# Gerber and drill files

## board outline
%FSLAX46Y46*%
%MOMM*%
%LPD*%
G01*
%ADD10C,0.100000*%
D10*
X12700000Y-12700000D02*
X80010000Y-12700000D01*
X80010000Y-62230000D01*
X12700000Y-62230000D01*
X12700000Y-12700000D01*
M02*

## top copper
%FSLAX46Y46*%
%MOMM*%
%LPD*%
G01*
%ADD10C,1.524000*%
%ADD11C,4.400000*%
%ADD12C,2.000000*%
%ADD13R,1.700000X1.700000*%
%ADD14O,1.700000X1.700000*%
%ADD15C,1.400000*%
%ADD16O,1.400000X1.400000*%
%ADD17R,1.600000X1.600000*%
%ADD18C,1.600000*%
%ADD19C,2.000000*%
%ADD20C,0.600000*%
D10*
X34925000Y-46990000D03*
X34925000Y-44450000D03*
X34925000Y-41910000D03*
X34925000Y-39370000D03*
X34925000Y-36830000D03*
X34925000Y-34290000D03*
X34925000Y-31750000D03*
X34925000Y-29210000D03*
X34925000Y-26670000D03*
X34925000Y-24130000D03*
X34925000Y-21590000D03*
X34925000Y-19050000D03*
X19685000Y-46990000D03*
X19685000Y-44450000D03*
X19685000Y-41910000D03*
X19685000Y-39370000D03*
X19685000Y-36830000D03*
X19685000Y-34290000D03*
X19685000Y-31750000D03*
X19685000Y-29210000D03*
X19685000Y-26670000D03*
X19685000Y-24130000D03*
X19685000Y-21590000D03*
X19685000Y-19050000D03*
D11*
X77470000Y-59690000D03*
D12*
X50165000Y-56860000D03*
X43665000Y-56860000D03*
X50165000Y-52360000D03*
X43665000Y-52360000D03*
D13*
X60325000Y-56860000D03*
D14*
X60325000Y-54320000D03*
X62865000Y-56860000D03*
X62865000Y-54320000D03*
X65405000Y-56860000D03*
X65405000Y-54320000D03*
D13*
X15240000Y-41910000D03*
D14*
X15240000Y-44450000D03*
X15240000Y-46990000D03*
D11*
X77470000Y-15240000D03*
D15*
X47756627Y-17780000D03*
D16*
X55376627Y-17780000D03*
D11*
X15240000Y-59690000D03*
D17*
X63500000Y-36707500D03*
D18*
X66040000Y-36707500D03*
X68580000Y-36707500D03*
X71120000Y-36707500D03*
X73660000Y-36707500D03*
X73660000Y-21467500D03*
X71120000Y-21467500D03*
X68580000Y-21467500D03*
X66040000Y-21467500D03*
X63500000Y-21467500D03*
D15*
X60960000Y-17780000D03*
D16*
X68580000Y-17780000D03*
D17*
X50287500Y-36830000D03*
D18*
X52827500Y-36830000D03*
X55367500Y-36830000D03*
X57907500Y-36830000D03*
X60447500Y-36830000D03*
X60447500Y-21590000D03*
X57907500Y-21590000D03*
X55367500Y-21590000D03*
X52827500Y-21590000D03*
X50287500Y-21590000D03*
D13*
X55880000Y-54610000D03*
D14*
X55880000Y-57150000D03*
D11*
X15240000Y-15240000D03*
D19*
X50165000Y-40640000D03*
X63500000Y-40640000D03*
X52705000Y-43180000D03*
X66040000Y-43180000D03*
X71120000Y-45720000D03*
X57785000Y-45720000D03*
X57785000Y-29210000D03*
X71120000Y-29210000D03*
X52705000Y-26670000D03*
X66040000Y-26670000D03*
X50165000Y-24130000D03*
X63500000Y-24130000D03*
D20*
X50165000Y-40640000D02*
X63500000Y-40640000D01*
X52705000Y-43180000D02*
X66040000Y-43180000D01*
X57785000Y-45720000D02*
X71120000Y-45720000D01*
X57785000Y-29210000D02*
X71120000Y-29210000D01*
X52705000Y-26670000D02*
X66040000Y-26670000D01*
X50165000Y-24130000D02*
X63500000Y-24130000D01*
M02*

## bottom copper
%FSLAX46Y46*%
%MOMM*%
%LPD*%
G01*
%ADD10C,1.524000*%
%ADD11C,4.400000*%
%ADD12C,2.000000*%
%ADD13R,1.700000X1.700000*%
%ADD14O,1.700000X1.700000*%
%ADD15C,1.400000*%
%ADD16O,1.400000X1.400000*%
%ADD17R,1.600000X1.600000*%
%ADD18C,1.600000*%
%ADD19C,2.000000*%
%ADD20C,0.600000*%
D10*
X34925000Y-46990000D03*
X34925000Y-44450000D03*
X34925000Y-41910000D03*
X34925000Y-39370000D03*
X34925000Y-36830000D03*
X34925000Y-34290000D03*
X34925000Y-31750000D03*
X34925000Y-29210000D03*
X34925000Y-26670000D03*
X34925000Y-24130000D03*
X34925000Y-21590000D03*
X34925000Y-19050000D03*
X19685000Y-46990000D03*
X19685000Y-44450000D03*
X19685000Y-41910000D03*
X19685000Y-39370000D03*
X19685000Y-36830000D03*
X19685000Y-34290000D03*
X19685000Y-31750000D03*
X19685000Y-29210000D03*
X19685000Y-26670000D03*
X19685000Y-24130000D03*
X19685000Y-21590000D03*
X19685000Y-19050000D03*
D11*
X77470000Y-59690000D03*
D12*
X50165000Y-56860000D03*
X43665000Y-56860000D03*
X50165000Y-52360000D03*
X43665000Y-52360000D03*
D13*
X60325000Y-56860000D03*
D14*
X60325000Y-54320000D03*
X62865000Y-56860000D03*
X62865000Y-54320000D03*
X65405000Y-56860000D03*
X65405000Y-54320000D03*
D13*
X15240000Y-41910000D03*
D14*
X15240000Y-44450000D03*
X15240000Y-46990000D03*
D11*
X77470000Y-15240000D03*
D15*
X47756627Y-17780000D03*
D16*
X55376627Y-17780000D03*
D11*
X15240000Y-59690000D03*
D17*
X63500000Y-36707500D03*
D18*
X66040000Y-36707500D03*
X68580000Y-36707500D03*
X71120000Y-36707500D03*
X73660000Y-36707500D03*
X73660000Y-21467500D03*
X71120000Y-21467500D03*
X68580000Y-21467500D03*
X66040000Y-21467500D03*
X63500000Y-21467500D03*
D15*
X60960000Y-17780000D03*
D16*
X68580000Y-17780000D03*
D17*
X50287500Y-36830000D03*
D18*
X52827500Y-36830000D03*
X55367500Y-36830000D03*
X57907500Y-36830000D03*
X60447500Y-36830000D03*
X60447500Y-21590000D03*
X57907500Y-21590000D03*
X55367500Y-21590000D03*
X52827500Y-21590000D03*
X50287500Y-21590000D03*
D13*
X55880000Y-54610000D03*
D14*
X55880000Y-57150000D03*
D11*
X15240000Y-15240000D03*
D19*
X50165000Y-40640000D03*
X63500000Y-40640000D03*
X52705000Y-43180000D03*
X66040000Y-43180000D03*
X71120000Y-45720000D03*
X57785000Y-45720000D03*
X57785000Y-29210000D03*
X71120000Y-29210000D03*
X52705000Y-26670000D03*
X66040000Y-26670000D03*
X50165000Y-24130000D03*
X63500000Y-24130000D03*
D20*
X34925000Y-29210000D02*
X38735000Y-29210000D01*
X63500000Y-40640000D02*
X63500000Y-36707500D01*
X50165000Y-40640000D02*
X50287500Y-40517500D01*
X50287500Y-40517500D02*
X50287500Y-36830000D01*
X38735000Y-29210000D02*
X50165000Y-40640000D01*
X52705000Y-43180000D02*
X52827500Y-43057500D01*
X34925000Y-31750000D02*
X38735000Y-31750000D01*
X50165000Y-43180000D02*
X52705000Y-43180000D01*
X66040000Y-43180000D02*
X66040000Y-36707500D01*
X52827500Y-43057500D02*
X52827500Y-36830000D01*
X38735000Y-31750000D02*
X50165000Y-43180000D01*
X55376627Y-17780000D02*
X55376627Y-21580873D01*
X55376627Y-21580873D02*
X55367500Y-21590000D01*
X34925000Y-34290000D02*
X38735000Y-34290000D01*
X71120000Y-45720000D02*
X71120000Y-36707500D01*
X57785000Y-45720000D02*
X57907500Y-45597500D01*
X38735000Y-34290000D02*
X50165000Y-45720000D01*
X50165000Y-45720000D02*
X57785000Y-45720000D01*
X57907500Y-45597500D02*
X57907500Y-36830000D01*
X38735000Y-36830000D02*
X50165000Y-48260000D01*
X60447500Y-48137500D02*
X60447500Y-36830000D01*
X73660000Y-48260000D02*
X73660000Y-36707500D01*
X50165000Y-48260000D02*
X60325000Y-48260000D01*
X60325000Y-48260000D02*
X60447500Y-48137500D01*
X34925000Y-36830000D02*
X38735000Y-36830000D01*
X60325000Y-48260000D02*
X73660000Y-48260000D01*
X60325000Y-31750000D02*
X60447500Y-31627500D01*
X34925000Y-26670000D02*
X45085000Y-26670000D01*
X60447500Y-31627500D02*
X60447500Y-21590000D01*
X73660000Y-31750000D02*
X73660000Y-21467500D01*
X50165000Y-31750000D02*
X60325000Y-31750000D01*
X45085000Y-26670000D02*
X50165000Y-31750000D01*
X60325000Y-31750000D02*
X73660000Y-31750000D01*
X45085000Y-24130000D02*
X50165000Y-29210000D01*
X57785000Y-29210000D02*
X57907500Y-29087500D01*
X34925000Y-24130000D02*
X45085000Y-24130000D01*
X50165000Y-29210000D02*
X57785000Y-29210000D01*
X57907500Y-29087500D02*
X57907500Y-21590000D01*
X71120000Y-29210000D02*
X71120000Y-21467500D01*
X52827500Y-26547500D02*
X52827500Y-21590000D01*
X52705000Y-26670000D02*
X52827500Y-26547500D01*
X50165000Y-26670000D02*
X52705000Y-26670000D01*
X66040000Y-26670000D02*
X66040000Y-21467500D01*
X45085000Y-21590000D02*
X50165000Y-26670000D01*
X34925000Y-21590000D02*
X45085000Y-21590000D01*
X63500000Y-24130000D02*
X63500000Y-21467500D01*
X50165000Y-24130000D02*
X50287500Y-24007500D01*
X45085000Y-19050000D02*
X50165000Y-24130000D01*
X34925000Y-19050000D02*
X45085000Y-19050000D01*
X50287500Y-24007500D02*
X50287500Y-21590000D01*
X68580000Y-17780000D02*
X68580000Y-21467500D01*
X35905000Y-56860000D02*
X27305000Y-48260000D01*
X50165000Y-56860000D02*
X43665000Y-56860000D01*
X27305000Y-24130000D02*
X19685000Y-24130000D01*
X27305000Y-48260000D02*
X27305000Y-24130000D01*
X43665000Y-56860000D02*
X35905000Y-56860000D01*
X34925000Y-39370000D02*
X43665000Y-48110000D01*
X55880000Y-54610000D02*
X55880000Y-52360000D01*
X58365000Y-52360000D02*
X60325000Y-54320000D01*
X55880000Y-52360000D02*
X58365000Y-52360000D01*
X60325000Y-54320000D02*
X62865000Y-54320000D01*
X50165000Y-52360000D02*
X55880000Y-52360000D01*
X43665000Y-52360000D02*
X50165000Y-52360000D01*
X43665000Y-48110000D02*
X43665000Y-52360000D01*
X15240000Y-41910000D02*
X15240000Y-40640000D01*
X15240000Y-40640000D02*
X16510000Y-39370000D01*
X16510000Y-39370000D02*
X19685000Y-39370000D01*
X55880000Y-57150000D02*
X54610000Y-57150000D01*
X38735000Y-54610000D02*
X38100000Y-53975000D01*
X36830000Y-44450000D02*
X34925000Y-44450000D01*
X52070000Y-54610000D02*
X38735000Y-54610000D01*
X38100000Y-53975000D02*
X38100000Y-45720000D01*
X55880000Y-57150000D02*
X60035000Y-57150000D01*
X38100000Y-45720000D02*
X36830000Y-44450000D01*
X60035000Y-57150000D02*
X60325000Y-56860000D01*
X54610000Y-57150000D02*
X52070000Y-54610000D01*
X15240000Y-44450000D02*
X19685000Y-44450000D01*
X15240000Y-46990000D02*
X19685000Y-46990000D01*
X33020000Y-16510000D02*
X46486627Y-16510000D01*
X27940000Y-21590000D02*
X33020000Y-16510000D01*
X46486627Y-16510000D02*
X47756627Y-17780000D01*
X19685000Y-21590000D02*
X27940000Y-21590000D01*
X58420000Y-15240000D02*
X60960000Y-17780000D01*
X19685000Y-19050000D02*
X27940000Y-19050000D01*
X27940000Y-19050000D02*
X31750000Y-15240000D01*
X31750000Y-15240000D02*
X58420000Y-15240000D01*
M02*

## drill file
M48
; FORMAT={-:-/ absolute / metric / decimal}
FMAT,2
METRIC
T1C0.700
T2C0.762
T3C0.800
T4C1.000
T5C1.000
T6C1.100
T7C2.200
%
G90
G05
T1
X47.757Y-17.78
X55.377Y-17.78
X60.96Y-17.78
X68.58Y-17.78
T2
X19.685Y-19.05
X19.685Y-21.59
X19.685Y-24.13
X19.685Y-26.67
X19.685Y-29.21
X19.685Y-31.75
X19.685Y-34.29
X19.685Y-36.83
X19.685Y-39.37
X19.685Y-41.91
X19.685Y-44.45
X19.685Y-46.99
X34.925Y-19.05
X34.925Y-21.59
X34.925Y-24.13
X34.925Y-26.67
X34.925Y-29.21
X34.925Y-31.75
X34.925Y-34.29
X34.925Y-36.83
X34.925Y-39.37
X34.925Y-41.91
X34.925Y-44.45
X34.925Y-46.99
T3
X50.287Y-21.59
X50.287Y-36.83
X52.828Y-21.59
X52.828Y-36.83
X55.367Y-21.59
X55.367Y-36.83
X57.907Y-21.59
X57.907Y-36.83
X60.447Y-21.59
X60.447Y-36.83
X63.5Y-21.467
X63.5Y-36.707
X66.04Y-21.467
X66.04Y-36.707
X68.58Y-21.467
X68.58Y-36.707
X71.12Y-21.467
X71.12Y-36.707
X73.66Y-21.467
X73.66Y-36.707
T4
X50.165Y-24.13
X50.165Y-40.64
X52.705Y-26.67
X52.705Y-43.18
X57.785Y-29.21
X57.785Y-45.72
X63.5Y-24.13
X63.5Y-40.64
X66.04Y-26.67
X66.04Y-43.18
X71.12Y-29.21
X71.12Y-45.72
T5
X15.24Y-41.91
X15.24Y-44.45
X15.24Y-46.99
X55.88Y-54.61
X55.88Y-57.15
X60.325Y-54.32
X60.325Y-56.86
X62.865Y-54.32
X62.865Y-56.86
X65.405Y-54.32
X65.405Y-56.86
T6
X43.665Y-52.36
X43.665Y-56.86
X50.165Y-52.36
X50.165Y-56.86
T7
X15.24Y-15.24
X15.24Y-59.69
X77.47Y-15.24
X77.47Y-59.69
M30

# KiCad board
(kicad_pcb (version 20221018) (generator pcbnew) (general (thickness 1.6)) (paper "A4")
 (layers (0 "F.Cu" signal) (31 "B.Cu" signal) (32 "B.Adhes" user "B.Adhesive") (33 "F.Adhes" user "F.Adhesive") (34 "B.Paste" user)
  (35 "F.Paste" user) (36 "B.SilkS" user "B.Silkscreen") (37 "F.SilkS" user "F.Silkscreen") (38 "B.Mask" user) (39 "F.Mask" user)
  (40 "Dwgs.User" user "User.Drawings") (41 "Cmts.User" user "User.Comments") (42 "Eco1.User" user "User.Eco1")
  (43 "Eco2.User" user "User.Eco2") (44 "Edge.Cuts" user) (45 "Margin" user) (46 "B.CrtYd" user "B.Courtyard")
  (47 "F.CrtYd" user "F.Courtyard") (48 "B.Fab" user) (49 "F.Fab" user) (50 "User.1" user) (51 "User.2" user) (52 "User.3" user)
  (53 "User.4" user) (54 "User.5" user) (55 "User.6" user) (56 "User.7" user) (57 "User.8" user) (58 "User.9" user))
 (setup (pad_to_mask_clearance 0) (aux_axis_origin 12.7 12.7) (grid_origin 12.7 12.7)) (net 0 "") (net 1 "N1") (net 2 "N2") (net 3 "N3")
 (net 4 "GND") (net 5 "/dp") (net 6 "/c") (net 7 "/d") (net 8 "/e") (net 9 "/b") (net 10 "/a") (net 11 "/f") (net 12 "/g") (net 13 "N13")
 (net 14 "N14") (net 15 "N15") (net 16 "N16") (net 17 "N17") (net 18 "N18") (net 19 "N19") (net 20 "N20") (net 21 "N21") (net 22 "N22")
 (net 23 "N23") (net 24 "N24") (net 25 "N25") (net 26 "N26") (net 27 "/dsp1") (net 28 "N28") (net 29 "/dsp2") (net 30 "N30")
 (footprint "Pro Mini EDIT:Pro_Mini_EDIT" (layer "F.Cu") (at 34.925 46.99 180)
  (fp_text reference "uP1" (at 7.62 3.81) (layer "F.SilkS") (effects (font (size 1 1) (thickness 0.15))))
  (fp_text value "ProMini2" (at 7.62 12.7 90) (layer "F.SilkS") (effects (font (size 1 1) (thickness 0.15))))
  (pad "7" thru_hole circle (at 0 0 180) (size 1.524 1.524) (drill 0.762) (layers "*.Cu" "*.Mask" "F.SilkS") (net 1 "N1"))
  (pad "8" thru_hole circle (at 0 2.54 180) (size 1.524 1.524) (drill 0.762) (layers "*.Cu" "*.Mask" "F.SilkS") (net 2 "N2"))
  (pad "9" thru_hole circle (at 0 5.08 180) (size 1.524 1.524) (drill 0.762) (layers "*.Cu" "*.Mask" "F.SilkS") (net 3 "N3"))
  (pad "10" thru_hole circle (at 0 7.62 180) (size 1.524 1.524) (drill 0.762) (layers "*.Cu" "*.Mask" "F.SilkS") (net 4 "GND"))
  (pad "11" thru_hole circle (at 0 10.16 180) (size 1.524 1.524) (drill 0.762) (layers "*.Cu" "*.Mask" "F.SilkS") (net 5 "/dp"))
  (pad "12" thru_hole circle (at 0 12.7 180) (size 1.524 1.524) (drill 0.762) (layers "*.Cu" "*.Mask" "F.SilkS") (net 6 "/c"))
  (pad "13" thru_hole circle (at 0 15.24 180) (size 1.524 1.524) (drill 0.762) (layers "*.Cu" "*.Mask" "F.SilkS") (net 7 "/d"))
  (pad "14" thru_hole circle (at 0 17.78 180) (size 1.524 1.524) (drill 0.762) (layers "*.Cu" "*.Mask" "F.SilkS") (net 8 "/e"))
  (pad "15" thru_hole circle (at 0 20.32 180) (size 1.524 1.524) (drill 0.762) (layers "*.Cu" "*.Mask" "F.SilkS") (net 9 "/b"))
  (pad "16" thru_hole circle (at 0 22.86 180) (size 1.524 1.524) (drill 0.762) (layers "*.Cu" "*.Mask" "F.SilkS") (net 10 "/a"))
  (pad "17" thru_hole circle (at 0 25.4 180) (size 1.524 1.524) (drill 0.762) (layers "*.Cu" "*.Mask" "F.SilkS") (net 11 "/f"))
  (pad "18" thru_hole circle (at 0 27.94 180) (size 1.524 1.524) (drill 0.762) (layers "*.Cu" "*.Mask" "F.SilkS") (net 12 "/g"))
  (pad "19" thru_hole circle (at 15.24 0 180) (size 1.524 1.524) (drill 0.762) (layers "*.Cu" "*.Mask" "F.SilkS") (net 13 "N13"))
  (pad "20" thru_hole circle (at 15.24 2.54 180) (size 1.524 1.524) (drill 0.762) (layers "*.Cu" "*.Mask" "F.SilkS") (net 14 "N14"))
  (pad "21" thru_hole circle (at 15.24 5.08 180) (size 1.524 1.524) (drill 0.762) (layers "*.Cu" "*.Mask" "F.SilkS") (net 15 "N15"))
  (pad "22" thru_hole circle (at 15.24 7.62 180) (size 1.524 1.524) (drill 0.762) (layers "*.Cu" "*.Mask" "F.SilkS") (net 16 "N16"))
  (pad "23" thru_hole circle (at 15.24 10.16 180) (size 1.524 1.524) (drill 0.762) (layers "*.Cu" "*.Mask" "F.SilkS") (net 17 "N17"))
  (pad "24" thru_hole circle (at 15.24 12.7 180) (size 1.524 1.524) (drill 0.762) (layers "*.Cu" "*.Mask" "F.SilkS") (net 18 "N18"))
  (pad "25" thru_hole circle (at 15.24 15.24 180) (size 1.524 1.524) (drill 0.762) (layers "*.Cu" "*.Mask" "F.SilkS") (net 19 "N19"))
  (pad "26" thru_hole circle (at 15.24 17.78 180) (size 1.524 1.524) (drill 0.762) (layers "*.Cu" "*.Mask" "F.SilkS") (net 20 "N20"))
  (pad "27" thru_hole circle (at 15.24 20.32 180) (size 1.524 1.524) (drill 0.762) (layers "*.Cu" "*.Mask" "F.SilkS") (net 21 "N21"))
  (pad "28" thru_hole circle (at 15.24 22.86 180) (size 1.524 1.524) (drill 0.762) (layers "*.Cu" "*.Mask" "F.SilkS") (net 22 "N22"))
  (pad "29" thru_hole circle (at 15.24 25.4 180) (size 1.524 1.524) (drill 0.762) (layers "*.Cu" "*.Mask" "F.SilkS") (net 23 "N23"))
  (pad "30" thru_hole circle (at 15.24 27.94 180) (size 1.524 1.524) (drill 0.762) (layers "*.Cu" "*.Mask" "F.SilkS") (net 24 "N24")))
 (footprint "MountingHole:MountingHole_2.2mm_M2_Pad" (layer "F.Cu") (at 77.47 59.69)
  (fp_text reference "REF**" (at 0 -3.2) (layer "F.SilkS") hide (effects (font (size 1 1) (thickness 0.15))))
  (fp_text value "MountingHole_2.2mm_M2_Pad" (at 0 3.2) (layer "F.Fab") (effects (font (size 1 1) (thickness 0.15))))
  (pad "1" thru_hole circle (at 0 0) (size 4.4 4.4) (drill 2.2) (layers "*.Cu" "*.Mask")))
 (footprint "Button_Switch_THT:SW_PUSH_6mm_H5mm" (layer "F.Cu") (at 50.165 56.86 180)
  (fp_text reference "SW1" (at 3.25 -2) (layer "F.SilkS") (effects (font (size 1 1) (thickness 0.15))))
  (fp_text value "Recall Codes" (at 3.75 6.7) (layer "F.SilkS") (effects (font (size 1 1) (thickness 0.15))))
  (pad "1" thru_hole circle (at 0 0 270) (size 2 2) (drill 1.1) (layers "*.Cu" "*.Mask") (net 22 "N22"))
  (pad "1" thru_hole circle (at 6.5 0 270) (size 2 2) (drill 1.1) (layers "*.Cu" "*.Mask") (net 22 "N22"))
  (pad "2" thru_hole circle (at 0 4.5 270) (size 2 2) (drill 1.1) (layers "*.Cu" "*.Mask") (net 4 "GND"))
  (pad "2" thru_hole circle (at 6.5 4.5 270) (size 2 2) (drill 1.1) (layers "*.Cu" "*.Mask") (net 4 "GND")))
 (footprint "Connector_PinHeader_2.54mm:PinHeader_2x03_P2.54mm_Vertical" (layer "F.Cu") (at 60.325 56.86 90)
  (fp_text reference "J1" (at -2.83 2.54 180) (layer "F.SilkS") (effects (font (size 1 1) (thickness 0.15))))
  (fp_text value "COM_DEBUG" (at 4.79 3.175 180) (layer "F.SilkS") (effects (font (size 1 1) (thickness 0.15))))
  (pad "1" thru_hole rect (at 0 0 90) (size 1.7 1.7) (drill 1) (layers "*.Cu" "*.Mask") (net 2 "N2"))
  (pad "2" thru_hole oval (at 2.54 0 90) (size 1.7 1.7) (drill 1) (layers "*.Cu" "*.Mask") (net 4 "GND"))
  (pad "3" thru_hole oval (at 0 2.54 90) (size 1.7 1.7) (drill 1) (layers "*.Cu" "*.Mask"))
  (pad "4" thru_hole oval (at 2.54 2.54 90) (size 1.7 1.7) (drill 1) (layers "*.Cu" "*.Mask") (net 4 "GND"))
  (pad "5" thru_hole oval (at 0 5.08 90) (size 1.7 1.7) (drill 1) (layers "*.Cu" "*.Mask") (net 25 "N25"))
  (pad "6" thru_hole oval (at 2.54 5.08 90) (size 1.7 1.7) (drill 1) (layers "*.Cu" "*.Mask") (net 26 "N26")))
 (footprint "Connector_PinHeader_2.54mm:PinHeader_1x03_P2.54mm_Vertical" (layer "F.Cu") (at 15.24 41.91)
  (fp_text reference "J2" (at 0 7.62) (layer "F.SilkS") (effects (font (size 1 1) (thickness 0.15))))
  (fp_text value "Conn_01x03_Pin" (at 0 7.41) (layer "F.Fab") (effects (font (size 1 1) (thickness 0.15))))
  (pad "1" thru_hole rect (at 0 0) (size 1.7 1.7) (drill 1) (layers "*.Cu" "*.Mask") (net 16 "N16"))
  (pad "2" thru_hole oval (at 0 2.54) (size 1.7 1.7) (drill 1) (layers "*.Cu" "*.Mask") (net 14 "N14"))
  (pad "3" thru_hole oval (at 0 5.08) (size 1.7 1.7) (drill 1) (layers "*.Cu" "*.Mask") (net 13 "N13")))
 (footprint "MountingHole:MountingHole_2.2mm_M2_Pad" (layer "F.Cu") (at 77.47 15.24)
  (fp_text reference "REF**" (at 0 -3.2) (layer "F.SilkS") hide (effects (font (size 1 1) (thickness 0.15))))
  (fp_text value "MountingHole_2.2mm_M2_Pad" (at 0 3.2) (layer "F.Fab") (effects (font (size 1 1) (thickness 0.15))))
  (pad "1" thru_hole circle (at 0 0) (size 4.4 4.4) (drill 2.2) (layers "*.Cu" "*.Mask")))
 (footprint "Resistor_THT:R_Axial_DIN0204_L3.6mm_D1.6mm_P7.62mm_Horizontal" (layer "F.Cu") (at 47.756627 17.78)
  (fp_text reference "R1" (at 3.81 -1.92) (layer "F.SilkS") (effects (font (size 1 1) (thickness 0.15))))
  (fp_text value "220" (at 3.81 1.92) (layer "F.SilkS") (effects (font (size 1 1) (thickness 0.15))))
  (pad "1" thru_hole circle (at 0 0) (size 1.4 1.4) (drill 0.7) (layers "*.Cu" "*.Mask") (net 23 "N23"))
  (pad "2" thru_hole oval (at 7.62 0) (size 1.4 1.4) (drill 0.7) (layers "*.Cu" "*.Mask") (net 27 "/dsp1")))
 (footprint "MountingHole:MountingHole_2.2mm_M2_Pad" (layer "F.Cu") (at 15.24 59.69)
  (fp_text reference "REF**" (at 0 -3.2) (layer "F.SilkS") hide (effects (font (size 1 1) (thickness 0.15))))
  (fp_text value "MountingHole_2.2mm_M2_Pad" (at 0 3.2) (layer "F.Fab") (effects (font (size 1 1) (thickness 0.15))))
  (pad "1" thru_hole circle (at 0 0) (size 4.4 4.4) (drill 2.2) (layers "*.Cu" "*.Mask")))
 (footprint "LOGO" (layer "F.Cu") (at 25.4 58.42)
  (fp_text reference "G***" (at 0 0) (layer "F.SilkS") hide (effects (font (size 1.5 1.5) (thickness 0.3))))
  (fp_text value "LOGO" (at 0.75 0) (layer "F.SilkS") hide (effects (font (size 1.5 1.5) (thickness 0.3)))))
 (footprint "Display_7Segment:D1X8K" (layer "F.Cu") (at 63.5 36.7075 90)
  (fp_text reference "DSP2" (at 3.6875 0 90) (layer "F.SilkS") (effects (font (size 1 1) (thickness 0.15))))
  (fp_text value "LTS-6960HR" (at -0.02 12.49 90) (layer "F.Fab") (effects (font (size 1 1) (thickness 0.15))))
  (pad "1" thru_hole rect (at 0 0) (size 1.6 1.6) (drill 0.8) (layers "*.Cu" "*.Mask") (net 8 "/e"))
  (pad "2" thru_hole circle (at 0 2.54) (size 1.6 1.6) (drill 0.8) (layers "*.Cu" "*.Mask") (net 7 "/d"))
  (pad "3" thru_hole circle (at 0 5.08) (size 1.6 1.6) (drill 0.8) (layers "*.Cu" "*.Mask") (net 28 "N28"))
  (pad "4" thru_hole circle (at 0 7.62) (size 1.6 1.6) (drill 0.8) (layers "*.Cu" "*.Mask") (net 6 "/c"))
  (pad "5" thru_hole circle (at 0 10.16) (size 1.6 1.6) (drill 0.8) (layers "*.Cu" "*.Mask") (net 5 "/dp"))
  (pad "6" thru_hole circle (at 15.24 10.16) (size 1.6 1.6) (drill 0.8) (layers "*.Cu" "*.Mask") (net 9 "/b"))
  (pad "7" thru_hole circle (at 15.24 7.62) (size 1.6 1.6) (drill 0.8) (layers "*.Cu" "*.Mask") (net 10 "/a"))
  (pad "8" thru_hole circle (at 15.24 5.08) (size 1.6 1.6) (drill 0.8) (layers "*.Cu" "*.Mask") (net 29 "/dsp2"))
  (pad "9" thru_hole circle (at 15.24 2.54) (size 1.6 1.6) (drill 0.8) (layers "*.Cu" "*.Mask") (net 11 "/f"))
  (pad "10" thru_hole circle (at 15.24 0) (size 1.6 1.6) (drill 0.8) (layers "*.Cu" "*.Mask") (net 12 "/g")))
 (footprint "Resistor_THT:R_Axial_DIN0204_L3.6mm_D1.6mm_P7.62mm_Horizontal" (layer "F.Cu") (at 60.96 17.78)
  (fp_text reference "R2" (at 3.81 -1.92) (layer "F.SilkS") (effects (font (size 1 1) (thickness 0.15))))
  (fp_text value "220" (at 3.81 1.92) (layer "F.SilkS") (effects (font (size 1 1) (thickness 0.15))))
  (pad "1" thru_hole circle (at 0 0) (size 1.4 1.4) (drill 0.7) (layers "*.Cu" "*.Mask") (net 24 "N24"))
  (pad "2" thru_hole oval (at 7.62 0) (size 1.4 1.4) (drill 0.7) (layers "*.Cu" "*.Mask") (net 29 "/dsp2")))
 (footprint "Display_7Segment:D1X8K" (layer "F.Cu") (at 50.2875 36.83 90)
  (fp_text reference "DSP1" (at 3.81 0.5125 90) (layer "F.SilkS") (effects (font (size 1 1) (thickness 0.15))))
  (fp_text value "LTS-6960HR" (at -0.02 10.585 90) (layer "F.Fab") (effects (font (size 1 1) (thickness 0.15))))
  (pad "1" thru_hole rect (at 0 0) (size 1.6 1.6) (drill 0.8) (layers "*.Cu" "*.Mask") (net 8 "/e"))
  (pad "2" thru_hole circle (at 0 2.54) (size 1.6 1.6) (drill 0.8) (layers "*.Cu" "*.Mask") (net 7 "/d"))
  (pad "3" thru_hole circle (at 0 5.08) (size 1.6 1.6) (drill 0.8) (layers "*.Cu" "*.Mask") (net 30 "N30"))
  (pad "4" thru_hole circle (at 0 7.62) (size 1.6 1.6) (drill 0.8) (layers "*.Cu" "*.Mask") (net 6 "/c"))
  (pad "5" thru_hole circle (at 0 10.16) (size 1.6 1.6) (drill 0.8) (layers "*.Cu" "*.Mask") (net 5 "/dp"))
  (pad "6" thru_hole circle (at 15.24 10.16) (size 1.6 1.6) (drill 0.8) (layers "*.Cu" "*.Mask") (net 9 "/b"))
  (pad "7" thru_hole circle (at 15.24 7.62) (size 1.6 1.6) (drill 0.8) (layers "*.Cu" "*.Mask") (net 10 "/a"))
  (pad "8" thru_hole circle (at 15.24 5.08) (size 1.6 1.6) (drill 0.8) (layers "*.Cu" "*.Mask") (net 27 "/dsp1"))
  (pad "9" thru_hole circle (at 15.24 2.54) (size 1.6 1.6) (drill 0.8) (layers "*.Cu" "*.Mask") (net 11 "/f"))
  (pad "10" thru_hole circle (at 15.24 0) (size 1.6 1.6) (drill 0.8) (layers "*.Cu" "*.Mask") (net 12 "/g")))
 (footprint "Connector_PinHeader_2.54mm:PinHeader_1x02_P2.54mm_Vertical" (layer "F.Cu") (at 55.88 54.61)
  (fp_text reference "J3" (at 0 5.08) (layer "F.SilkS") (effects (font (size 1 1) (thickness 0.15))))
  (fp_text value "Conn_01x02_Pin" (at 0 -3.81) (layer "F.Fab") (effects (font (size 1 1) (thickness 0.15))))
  (pad "1" thru_hole rect (at 0 0) (size 1.7 1.7) (drill 1) (layers "*.Cu" "*.Mask") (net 4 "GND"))
  (pad "2" thru_hole oval (at 0 2.54) (size 1.7 1.7) (drill 1) (layers "*.Cu" "*.Mask") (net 2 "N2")))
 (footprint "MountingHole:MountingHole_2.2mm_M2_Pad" (layer "F.Cu") (at 15.24 15.24)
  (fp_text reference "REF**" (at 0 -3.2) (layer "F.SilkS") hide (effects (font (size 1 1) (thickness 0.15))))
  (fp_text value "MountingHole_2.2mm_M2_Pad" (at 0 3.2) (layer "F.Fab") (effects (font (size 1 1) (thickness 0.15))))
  (pad "1" thru_hole circle (at 0 0) (size 4.4 4.4) (drill 2.2) (layers "*.Cu" "*.Mask")))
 (gr_rect (start 12.7 12.7) (end 80.01 62.23) (stroke (width 0.1) (type default)) (fill none) (layer "Edge.Cuts"))
 (segment (start 50.165 40.64) (end 63.5 40.64) (width 0.6) (layer "F.Cu") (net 8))
 (via (at 50.165 40.64) (size 2) (drill 1) (layers "F.Cu" "B.Cu") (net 8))
 (via (at 63.5 40.64) (size 2) (drill 1) (layers "F.Cu" "B.Cu") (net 8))
 (segment (start 34.925 29.21) (end 38.735 29.21) (width 0.6) (layer "B.Cu") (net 8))
 (segment (start 63.5 40.64) (end 63.5 36.7075) (width 0.6) (layer "B.Cu") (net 8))
 (segment (start 50.165 40.64) (end 50.2875 40.5175) (width 0.6) (layer "B.Cu") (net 8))
 (segment (start 50.2875 40.5175) (end 50.2875 36.83) (width 0.6) (layer "B.Cu") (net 8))
 (segment (start 38.735 29.21) (end 50.165 40.64) (width 0.6) (layer "B.Cu") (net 8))
 (segment (start 52.705 43.18) (end 66.04 43.18) (width 0.6) (layer "F.Cu") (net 7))
 (via (at 52.705 43.18) (size 2) (drill 1) (layers "F.Cu" "B.Cu") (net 7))
 (via (at 66.04 43.18) (size 2) (drill 1) (layers "F.Cu" "B.Cu") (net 7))
 (segment (start 52.705 43.18) (end 52.8275 43.0575) (width 0.6) (layer "B.Cu") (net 7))
 (segment (start 34.925 31.75) (end 38.735 31.75) (width 0.6) (layer "B.Cu") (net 7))
 (segment (start 50.165 43.18) (end 52.705 43.18) (width 0.6) (layer "B.Cu") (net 7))
 (segment (start 66.04 43.18) (end 66.04 36.7075) (width 0.6) (layer "B.Cu") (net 7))
 (segment (start 52.8275 43.0575) (end 52.8275 36.83) (width 0.6) (layer "B.Cu") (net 7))
 (segment (start 38.735 31.75) (end 50.165 43.18) (width 0.6) (layer "B.Cu") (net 7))
 (segment (start 55.376627 17.78) (end 55.376627 21.580873) (width 0.6) (layer "B.Cu") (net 27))
 (segment (start 55.376627 21.580873) (end 55.3675 21.59) (width 0.6) (layer "B.Cu") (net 27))
 (segment (start 57.785 45.72) (end 71.12 45.72) (width 0.6) (layer "F.Cu") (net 6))
 (via (at 71.12 45.72) (size 2) (drill 1) (layers "F.Cu" "B.Cu") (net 6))
 (via (at 57.785 45.72) (size 2) (drill 1) (layers "F.Cu" "B.Cu") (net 6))
 (segment (start 34.925 34.29) (end 38.735 34.29) (width 0.6) (layer "B.Cu") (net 6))
 (segment (start 71.12 45.72) (end 71.12 36.7075) (width 0.6) (layer "B.Cu") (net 6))
 (segment (start 57.785 45.72) (end 57.9075 45.5975) (width 0.6) (layer "B.Cu") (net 6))
 (segment (start 38.735 34.29) (end 50.165 45.72) (width 0.6) (layer "B.Cu") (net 6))
 (segment (start 50.165 45.72) (end 57.785 45.72) (width 0.6) (layer "B.Cu") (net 6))
 (segment (start 57.9075 45.5975) (end 57.9075 36.83) (width 0.6) (layer "B.Cu") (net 6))
 (segment (start 38.735 36.83) (end 50.165 48.26) (width 0.6) (layer "B.Cu") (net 5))
 (segment (start 60.4475 48.1375) (end 60.4475 36.83) (width 0.6) (layer "B.Cu") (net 5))
 (segment (start 73.66 48.26) (end 73.66 36.7075) (width 0.6) (layer "B.Cu") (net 5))
 (segment (start 50.165 48.26) (end 60.325 48.26) (width 0.6) (layer "B.Cu") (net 5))
 (segment (start 60.325 48.26) (end 60.4475 48.1375) (width 0.6) (layer "B.Cu") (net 5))
 (segment (start 34.925 36.83) (end 38.735 36.83) (width 0.6) (layer "B.Cu") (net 5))
 (segment (start 60.325 48.26) (end 73.66 48.26) (width 0.6) (layer "B.Cu") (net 5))
 (segment (start 60.325 31.75) (end 60.4475 31.6275) (width 0.6) (layer "B.Cu") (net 9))
 (segment (start 34.925 26.67) (end 45.085 26.67) (width 0.6) (layer "B.Cu") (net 9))
 (segment (start 60.4475 31.6275) (end 60.4475 21.59) (width 0.6) (layer "B.Cu") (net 9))
 (segment (start 73.66 31.75) (end 73.66 21.4675) (width 0.6) (layer "B.Cu") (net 9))
 (segment (start 50.165 31.75) (end 60.325 31.75) (width 0.6) (layer "B.Cu") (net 9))
 (segment (start 45.085 26.67) (end 50.165 31.75) (width 0.6) (layer "B.Cu") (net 9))
 (segment (start 60.325 31.75) (end 73.66 31.75) (width 0.6) (layer "B.Cu") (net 9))
 (segment (start 57.785 29.21) (end 71.12 29.21) (width 0.6) (layer "F.Cu") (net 10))
 (via (at 57.785 29.21) (size 2) (drill 1) (layers "F.Cu" "B.Cu") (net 10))
 (via (at 71.12 29.21) (size 2) (drill 1) (layers "F.Cu" "B.Cu") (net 10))
 (segment (start 45.085 24.13) (end 50.165 29.21) (width 0.6) (layer "B.Cu") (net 10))
 (segment (start 57.785 29.21) (end 57.9075 29.0875) (width 0.6) (layer "B.Cu") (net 10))
 (segment (start 34.925 24.13) (end 45.085 24.13) (width 0.6) (layer "B.Cu") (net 10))
 (segment (start 50.165 29.21) (end 57.785 29.21) (width 0.6) (layer "B.Cu") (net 10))
 (segment (start 57.9075 29.0875) (end 57.9075 21.59) (width 0.6) (layer "B.Cu") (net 10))
 (segment (start 71.12 29.21) (end 71.12 21.4675) (width 0.6) (layer "B.Cu") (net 10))
 (segment (start 52.705 26.67) (end 66.04 26.67) (width 0.6) (layer "F.Cu") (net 11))
 (via (at 52.705 26.67) (size 2) (drill 1) (layers "F.Cu" "B.Cu") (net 11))
 (via (at 66.04 26.67) (size 2) (drill 1) (layers "F.Cu" "B.Cu") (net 11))
 (segment (start 52.8275 26.5475) (end 52.8275 21.59) (width 0.6) (layer "B.Cu") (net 11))
 (segment (start 52.705 26.67) (end 52.8275 26.5475) (width 0.6) (layer "B.Cu") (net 11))
 (segment (start 50.165 26.67) (end 52.705 26.67) (width 0.6) (layer "B.Cu") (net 11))
 (segment (start 66.04 26.67) (end 66.04 21.4675) (width 0.6) (layer "B.Cu") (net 11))
 (segment (start 45.085 21.59) (end 50.165 26.67) (width 0.6) (layer "B.Cu") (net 11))
 (segment (start 34.925 21.59) (end 45.085 21.59) (width 0.6) (layer "B.Cu") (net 11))
 (segment (start 50.165 24.13) (end 63.5 24.13) (width 0.6) (layer "F.Cu") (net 12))
 (via (at 50.165 24.13) (size 2) (drill 1) (layers "F.Cu" "B.Cu") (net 12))
 (via (at 63.5 24.13) (size 2) (drill 1) (layers "F.Cu" "B.Cu") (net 12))
 (segment (start 63.5 24.13) (end 63.5 21.4675) (width 0.6) (layer "B.Cu") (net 12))
 (segment (start 50.165 24.13) (end 50.2875 24.0075) (width 0.6) (layer "B.Cu") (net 12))
 (segment (start 45.085 19.05) (end 50.165 24.13) (width 0.6) (layer "B.Cu") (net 12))
 (segment (start 34.925 19.05) (end 45.085 19.05) (width 0.6) (layer "B.Cu") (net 12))
 (segment (start 50.2875 24.0075) (end 50.2875 21.59) (width 0.6) (layer "B.Cu") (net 12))
 (segment (start 68.58 17.78) (end 68.58 21.4675) (width 0.6) (layer "B.Cu") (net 29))
 (segment (start 35.905 56.86) (end 27.305 48.26) (width 0.6) (layer "B.Cu") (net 22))
 (segment (start 50.165 56.86) (end 43.665 56.86) (width 0.6) (layer "B.Cu") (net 22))
 (segment (start 27.305 24.13) (end 19.685 24.13) (width 0.6) (layer "B.Cu") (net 22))
 (segment (start 27.305 48.26) (end 27.305 24.13) (width 0.6) (layer "B.Cu") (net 22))
 (segment (start 43.665 56.86) (end 35.905 56.86) (width 0.6) (layer "B.Cu") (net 22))
 (segment (start 34.925 39.37) (end 43.665 48.11) (width 0.6) (layer "B.Cu") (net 4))
 (segment (start 55.88 54.61) (end 55.88 52.36) (width 0.6) (layer "B.Cu") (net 4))
 (segment (start 58.365 52.36) (end 60.325 54.32) (width 0.6) (layer "B.Cu") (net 4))
 (segment (start 55.88 52.36) (end 58.365 52.36) (width 0.6) (layer "B.Cu") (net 4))
 (segment (start 60.325 54.32) (end 62.865 54.32) (width 0.6) (layer "B.Cu") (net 4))
 (segment (start 50.165 52.36) (end 55.88 52.36) (width 0.6) (layer "B.Cu") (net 4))
 (segment (start 43.665 52.36) (end 50.165 52.36) (width 0.6) (layer "B.Cu") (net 4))
 (segment (start 43.665 48.11) (end 43.665 52.36) (width 0.6) (layer "B.Cu") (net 4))
 (segment (start 15.24 41.91) (end 15.24 40.64) (width 0.6) (layer "B.Cu") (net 16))
 (segment (start 15.24 40.64) (end 16.51 39.37) (width 0.6) (layer "B.Cu") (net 16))
 (segment (start 16.51 39.37) (end 19.685 39.37) (width 0.6) (layer "B.Cu") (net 16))
 (segment (start 55.88 57.15) (end 54.61 57.15) (width 0.6) (layer "B.Cu") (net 2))
 (segment (start 38.735 54.61) (end 38.1 53.975) (width 0.6) (layer "B.Cu") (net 2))
 (segment (start 36.83 44.45) (end 34.925 44.45) (width 0.6) (layer "B.Cu") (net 2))
 (segment (start 52.07 54.61) (end 38.735 54.61) (width 0.6) (layer "B.Cu") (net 2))
 (segment (start 38.1 53.975) (end 38.1 45.72) (width 0.6) (layer "B.Cu") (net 2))
 (segment (start 55.88 57.15) (end 60.035 57.15) (width 0.6) (layer "B.Cu") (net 2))
 (segment (start 38.1 45.72) (end 36.83 44.45) (width 0.6) (layer "B.Cu") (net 2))
 (segment (start 60.035 57.15) (end 60.325 56.86) (width 0.6) (layer "B.Cu") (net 2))
 (segment (start 54.61 57.15) (end 52.07 54.61) (width 0.6) (layer "B.Cu") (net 2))
 (segment (start 15.24 44.45) (end 19.685 44.45) (width 0.6) (layer "B.Cu") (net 14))
 (segment (start 15.24 46.99) (end 19.685 46.99) (width 0.6) (layer "B.Cu") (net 13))
 (segment (start 33.02 16.51) (end 46.486627 16.51) (width 0.6) (layer "B.Cu") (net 23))
 (segment (start 27.94 21.59) (end 33.02 16.51) (width 0.6) (layer "B.Cu") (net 23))
 (segment (start 46.486627 16.51) (end 47.756627 17.78) (width 0.6) (layer "B.Cu") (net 23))
 (segment (start 19.685 21.59) (end 27.94 21.59) (width 0.6) (layer "B.Cu") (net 23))
 (segment (start 58.42 15.24) (end 60.96 17.78) (width 0.6) (layer "B.Cu") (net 24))
 (segment (start 19.685 19.05) (end 27.94 19.05) (width 0.6) (layer "B.Cu") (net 24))
 (segment (start 27.94 19.05) (end 31.75 15.24) (width 0.6) (layer "B.Cu") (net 24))
 (segment (start 31.75 15.24) (end 58.42 15.24) (width 0.6) (layer "B.Cu") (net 24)))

